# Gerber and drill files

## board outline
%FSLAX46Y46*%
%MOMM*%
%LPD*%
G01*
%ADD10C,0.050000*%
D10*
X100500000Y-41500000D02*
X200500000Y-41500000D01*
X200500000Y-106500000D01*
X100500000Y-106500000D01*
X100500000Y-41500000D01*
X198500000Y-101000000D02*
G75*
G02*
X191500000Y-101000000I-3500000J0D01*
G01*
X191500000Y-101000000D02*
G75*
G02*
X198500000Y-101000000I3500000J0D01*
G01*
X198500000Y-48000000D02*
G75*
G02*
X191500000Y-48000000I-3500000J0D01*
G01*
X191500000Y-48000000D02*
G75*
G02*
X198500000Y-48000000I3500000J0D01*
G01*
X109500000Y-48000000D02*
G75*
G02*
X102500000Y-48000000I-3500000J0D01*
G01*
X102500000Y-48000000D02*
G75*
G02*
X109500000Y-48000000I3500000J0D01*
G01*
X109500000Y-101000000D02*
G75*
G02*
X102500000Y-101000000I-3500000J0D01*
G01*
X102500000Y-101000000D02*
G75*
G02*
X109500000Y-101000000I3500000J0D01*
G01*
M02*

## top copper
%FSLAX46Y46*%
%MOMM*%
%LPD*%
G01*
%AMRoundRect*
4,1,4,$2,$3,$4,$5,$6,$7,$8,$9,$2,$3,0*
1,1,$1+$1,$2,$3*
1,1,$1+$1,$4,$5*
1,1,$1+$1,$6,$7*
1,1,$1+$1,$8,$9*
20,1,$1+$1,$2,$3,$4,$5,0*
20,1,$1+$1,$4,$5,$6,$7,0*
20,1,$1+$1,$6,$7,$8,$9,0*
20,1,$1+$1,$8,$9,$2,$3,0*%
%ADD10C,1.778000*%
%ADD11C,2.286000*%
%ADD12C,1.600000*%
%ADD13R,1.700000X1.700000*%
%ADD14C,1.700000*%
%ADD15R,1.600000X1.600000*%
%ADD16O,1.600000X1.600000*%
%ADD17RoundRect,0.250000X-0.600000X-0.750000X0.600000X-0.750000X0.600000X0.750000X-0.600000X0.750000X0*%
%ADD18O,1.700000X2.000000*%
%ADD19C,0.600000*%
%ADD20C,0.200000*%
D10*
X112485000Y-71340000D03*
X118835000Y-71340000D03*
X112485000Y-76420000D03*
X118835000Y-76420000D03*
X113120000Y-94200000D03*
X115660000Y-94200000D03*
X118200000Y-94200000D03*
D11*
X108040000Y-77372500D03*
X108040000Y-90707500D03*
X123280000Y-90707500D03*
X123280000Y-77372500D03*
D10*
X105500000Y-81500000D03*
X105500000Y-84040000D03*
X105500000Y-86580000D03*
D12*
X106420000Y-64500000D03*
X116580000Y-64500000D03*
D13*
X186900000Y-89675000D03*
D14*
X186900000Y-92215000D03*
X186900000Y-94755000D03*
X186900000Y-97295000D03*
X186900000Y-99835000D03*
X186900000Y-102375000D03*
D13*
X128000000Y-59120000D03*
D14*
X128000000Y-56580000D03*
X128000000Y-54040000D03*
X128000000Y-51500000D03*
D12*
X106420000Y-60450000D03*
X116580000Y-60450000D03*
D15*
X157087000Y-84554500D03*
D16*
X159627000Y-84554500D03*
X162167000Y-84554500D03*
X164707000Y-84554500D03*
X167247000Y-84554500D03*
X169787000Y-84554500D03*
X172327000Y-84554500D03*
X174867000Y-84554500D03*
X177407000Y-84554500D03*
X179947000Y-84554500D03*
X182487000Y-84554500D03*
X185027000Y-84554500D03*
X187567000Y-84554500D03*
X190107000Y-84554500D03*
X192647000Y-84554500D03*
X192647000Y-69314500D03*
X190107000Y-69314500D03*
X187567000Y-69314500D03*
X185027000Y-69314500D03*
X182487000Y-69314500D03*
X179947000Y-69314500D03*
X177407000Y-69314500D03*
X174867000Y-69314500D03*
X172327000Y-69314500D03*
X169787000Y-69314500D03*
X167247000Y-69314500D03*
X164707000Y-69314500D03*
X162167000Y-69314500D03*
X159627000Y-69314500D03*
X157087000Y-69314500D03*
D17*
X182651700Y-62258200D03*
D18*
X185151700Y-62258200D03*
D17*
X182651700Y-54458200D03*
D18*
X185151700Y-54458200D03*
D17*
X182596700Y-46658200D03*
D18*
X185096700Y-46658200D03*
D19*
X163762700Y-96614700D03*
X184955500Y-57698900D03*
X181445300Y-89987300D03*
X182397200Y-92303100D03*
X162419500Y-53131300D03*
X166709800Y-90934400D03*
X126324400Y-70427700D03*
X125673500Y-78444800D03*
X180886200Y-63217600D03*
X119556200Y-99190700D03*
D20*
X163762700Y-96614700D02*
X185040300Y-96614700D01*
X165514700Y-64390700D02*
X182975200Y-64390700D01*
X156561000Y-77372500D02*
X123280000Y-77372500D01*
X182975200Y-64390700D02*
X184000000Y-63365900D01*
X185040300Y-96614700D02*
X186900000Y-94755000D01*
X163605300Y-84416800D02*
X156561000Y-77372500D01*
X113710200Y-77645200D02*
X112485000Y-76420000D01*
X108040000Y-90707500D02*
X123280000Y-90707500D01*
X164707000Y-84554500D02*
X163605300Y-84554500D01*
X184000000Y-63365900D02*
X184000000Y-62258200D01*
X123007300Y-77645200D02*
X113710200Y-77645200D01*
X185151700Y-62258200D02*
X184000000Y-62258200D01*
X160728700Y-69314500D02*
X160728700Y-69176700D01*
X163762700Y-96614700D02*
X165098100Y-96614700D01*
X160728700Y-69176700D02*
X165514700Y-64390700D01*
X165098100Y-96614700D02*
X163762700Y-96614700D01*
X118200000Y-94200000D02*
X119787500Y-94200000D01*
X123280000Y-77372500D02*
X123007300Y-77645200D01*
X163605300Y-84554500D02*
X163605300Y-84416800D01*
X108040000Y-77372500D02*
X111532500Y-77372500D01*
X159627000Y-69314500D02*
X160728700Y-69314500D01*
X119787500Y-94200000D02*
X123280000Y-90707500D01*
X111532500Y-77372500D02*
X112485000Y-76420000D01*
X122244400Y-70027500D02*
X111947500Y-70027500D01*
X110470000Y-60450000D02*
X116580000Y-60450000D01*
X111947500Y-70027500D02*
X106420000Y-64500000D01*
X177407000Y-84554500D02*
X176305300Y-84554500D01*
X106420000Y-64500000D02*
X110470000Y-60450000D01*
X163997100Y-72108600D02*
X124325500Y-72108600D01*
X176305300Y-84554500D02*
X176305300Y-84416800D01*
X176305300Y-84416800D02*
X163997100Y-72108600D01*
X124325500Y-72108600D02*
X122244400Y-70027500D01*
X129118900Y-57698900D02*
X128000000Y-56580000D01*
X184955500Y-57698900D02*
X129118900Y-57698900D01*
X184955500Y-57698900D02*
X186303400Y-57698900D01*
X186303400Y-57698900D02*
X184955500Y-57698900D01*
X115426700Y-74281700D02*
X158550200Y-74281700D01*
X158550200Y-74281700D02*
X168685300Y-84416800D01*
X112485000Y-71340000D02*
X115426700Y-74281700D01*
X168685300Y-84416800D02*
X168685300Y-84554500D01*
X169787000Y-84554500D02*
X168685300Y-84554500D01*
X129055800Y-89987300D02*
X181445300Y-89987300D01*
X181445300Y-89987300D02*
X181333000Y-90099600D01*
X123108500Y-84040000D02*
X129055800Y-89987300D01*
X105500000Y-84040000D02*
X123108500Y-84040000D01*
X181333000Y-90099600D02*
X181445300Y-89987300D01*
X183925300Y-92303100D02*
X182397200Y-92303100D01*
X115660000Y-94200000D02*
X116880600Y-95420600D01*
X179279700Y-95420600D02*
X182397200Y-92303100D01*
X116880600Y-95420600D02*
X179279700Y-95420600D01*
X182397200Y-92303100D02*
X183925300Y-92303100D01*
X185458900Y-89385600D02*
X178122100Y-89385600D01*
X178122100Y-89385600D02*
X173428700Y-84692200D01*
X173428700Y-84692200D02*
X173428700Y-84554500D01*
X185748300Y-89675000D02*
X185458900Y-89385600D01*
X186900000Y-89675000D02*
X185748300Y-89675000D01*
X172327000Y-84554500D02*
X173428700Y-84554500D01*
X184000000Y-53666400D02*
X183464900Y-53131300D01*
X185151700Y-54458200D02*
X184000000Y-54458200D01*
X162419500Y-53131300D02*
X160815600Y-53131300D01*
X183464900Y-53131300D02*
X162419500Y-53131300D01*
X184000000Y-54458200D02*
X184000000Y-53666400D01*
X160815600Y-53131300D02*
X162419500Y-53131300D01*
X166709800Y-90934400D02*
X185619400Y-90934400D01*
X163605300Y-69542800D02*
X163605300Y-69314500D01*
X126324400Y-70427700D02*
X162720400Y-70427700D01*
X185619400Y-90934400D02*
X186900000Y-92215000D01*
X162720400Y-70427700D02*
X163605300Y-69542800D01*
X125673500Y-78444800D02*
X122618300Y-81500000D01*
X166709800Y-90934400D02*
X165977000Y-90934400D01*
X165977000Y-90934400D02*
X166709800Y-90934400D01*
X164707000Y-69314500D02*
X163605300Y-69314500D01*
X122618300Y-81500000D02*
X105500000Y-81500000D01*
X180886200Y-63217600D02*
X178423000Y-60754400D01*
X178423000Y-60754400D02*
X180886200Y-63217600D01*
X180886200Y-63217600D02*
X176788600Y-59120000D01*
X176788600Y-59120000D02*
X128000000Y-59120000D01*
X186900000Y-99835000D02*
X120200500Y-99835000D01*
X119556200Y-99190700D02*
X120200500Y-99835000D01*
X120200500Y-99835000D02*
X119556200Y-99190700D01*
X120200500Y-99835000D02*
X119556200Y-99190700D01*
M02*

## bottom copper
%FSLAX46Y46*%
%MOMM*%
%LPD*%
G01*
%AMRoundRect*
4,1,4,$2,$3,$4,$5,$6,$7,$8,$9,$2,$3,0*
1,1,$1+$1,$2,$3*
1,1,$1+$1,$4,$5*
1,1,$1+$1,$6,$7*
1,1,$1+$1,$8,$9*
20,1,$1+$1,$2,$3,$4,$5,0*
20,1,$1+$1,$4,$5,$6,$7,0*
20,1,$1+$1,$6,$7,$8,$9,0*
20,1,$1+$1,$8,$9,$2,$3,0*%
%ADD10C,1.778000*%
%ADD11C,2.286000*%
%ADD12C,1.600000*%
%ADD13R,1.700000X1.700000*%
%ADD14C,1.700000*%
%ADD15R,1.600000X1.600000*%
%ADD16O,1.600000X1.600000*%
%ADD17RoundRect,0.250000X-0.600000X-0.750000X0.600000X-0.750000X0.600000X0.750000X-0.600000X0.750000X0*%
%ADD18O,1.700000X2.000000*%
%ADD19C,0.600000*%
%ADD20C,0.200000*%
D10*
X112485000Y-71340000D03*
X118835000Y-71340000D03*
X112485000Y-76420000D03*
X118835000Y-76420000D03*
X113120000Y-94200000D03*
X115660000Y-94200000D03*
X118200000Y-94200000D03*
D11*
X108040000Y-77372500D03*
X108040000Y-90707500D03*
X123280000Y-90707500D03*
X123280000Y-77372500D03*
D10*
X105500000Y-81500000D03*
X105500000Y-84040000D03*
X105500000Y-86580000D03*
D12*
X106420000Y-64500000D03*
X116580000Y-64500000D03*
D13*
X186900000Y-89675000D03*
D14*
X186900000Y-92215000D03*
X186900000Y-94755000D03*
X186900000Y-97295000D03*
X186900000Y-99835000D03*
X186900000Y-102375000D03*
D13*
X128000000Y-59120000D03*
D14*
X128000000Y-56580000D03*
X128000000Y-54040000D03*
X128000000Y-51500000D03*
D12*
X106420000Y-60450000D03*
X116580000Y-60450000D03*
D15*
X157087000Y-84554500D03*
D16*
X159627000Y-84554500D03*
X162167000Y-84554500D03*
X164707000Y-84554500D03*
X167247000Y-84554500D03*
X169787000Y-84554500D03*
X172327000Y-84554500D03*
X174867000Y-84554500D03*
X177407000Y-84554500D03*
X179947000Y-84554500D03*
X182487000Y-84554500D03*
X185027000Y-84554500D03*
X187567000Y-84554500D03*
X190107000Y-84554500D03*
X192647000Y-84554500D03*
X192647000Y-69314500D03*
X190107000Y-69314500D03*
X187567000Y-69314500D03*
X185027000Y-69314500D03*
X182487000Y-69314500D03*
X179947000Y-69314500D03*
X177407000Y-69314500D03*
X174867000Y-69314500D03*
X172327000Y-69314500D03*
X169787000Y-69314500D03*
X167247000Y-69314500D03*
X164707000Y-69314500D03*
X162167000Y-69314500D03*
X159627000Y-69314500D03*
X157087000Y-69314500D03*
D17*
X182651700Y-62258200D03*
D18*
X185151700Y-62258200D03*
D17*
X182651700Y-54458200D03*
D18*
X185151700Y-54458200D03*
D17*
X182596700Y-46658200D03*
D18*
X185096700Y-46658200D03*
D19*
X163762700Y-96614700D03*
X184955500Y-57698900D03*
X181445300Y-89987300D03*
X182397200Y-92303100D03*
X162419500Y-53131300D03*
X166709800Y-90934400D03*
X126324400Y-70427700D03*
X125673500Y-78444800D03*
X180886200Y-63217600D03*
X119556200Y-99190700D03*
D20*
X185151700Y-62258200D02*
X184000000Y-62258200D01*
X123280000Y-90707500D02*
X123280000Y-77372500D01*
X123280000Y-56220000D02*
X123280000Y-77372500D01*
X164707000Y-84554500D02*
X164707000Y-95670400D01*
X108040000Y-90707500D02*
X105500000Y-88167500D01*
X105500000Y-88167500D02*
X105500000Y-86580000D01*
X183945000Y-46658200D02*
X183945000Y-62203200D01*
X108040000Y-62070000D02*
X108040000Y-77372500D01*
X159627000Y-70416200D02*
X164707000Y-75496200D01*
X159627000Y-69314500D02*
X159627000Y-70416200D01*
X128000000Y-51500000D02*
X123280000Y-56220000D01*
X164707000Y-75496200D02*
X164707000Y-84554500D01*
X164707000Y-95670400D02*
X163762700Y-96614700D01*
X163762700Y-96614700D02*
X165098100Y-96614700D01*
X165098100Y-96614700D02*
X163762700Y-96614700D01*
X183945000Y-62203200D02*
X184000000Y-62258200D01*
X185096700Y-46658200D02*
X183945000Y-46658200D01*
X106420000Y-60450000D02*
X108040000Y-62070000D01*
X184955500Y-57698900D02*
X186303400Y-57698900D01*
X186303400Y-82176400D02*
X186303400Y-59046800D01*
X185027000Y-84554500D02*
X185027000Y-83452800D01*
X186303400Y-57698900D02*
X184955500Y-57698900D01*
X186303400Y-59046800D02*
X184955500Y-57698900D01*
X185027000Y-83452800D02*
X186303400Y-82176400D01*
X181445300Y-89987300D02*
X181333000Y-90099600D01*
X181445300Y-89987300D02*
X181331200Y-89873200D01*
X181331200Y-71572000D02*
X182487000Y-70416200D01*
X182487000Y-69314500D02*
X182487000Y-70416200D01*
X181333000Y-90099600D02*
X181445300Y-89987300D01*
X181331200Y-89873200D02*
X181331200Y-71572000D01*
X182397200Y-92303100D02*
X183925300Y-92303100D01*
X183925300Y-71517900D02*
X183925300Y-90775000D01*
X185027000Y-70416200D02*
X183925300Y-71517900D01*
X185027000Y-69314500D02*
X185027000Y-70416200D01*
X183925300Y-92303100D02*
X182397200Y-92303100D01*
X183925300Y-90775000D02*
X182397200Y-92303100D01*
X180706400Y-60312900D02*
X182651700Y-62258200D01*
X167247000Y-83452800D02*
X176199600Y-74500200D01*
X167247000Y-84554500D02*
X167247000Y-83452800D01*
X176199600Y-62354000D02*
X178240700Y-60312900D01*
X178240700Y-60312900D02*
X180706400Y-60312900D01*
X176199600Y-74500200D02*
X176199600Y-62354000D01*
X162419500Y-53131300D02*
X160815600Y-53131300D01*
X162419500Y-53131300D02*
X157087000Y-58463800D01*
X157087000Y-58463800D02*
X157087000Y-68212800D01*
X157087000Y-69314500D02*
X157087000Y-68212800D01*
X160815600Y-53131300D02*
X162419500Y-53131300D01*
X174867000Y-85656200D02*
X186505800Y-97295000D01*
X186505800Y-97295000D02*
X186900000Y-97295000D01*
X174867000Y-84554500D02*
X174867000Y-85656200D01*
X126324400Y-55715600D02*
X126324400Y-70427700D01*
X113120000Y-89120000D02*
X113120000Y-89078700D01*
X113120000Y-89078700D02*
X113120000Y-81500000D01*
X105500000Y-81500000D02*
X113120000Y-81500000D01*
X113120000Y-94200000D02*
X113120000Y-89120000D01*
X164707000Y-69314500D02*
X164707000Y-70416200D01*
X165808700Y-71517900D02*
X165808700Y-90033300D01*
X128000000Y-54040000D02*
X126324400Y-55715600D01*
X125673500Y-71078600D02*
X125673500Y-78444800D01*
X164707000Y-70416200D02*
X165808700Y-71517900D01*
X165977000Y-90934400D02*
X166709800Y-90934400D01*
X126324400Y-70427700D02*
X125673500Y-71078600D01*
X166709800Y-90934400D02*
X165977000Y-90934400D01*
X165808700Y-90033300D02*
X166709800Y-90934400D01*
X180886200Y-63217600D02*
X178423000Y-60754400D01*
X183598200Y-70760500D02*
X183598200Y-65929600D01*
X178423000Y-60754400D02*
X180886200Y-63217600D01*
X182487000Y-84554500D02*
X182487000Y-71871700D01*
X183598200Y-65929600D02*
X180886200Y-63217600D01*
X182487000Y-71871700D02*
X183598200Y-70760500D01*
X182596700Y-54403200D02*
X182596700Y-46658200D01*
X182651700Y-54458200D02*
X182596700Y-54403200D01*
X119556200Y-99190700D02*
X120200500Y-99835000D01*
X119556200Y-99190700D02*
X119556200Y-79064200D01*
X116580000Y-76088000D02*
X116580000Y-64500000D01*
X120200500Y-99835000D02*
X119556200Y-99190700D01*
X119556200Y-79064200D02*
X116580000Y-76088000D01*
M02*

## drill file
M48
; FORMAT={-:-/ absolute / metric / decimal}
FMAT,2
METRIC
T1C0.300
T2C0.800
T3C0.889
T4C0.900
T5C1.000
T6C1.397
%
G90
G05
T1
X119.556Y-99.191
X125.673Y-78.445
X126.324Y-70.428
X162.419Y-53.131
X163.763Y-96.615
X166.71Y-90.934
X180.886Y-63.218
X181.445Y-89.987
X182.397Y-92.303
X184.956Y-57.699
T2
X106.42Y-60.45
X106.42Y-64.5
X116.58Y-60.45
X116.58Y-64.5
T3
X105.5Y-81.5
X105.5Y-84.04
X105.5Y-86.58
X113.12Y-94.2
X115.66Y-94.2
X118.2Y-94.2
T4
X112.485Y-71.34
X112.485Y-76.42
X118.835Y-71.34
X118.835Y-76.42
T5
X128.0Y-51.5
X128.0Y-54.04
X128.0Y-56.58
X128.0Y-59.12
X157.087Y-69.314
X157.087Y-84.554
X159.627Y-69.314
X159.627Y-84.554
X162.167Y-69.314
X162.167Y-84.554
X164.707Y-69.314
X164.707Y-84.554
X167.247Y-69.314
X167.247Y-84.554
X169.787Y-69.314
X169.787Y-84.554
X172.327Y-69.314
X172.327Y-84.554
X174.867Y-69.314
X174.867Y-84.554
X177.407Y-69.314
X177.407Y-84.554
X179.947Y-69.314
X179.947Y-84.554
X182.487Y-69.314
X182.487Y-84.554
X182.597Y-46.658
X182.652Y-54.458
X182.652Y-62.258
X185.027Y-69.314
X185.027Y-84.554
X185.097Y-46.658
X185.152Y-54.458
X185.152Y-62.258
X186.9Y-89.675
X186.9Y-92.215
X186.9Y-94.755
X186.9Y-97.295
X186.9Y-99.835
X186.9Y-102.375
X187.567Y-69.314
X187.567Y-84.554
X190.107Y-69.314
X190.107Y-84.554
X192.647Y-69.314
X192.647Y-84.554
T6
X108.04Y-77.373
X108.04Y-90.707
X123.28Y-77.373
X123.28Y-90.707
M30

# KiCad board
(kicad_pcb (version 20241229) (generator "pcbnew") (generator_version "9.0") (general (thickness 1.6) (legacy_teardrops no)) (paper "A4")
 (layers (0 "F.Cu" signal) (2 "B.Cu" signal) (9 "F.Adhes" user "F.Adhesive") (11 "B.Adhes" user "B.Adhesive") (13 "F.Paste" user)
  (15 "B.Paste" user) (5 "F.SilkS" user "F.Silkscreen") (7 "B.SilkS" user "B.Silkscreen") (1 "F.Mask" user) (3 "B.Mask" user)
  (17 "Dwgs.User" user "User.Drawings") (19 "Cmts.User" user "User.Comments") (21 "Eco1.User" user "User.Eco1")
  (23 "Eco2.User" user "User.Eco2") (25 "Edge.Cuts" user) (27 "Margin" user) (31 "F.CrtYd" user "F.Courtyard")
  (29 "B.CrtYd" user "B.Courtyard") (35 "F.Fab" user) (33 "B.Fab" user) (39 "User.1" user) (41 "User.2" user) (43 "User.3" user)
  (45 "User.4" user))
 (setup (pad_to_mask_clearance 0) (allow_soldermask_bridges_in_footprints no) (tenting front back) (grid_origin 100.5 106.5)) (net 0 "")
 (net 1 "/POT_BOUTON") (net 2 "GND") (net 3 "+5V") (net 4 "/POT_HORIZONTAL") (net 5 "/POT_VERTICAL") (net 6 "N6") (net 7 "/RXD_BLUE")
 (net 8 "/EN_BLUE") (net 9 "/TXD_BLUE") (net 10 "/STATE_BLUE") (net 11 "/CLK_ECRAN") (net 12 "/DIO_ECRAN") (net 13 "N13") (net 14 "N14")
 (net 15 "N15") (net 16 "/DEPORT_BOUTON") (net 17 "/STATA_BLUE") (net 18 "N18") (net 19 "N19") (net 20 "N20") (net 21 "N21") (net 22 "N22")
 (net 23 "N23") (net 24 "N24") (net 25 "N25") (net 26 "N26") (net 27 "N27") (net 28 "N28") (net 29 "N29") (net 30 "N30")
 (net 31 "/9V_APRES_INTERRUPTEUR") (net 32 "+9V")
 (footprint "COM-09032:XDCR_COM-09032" (layer "F.Cu") (at 115.66 84.04)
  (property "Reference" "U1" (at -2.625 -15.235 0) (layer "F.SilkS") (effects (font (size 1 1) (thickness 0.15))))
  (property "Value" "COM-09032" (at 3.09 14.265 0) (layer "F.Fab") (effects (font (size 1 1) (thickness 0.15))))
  (pad "B1A" thru_hole circle (at -3.175 -12.7) (size 1.778 1.778) (drill 0.9) (layers "*.Cu" "*.Mask") (remove_unused_layers no)
   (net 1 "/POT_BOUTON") (solder_mask_margin 0.102))
  (pad "B1B" thru_hole circle (at 3.175 -12.7) (size 1.778 1.778) (drill 0.9) (layers "*.Cu" "*.Mask") (remove_unused_layers no)
   (solder_mask_margin 0.102))
  (pad "B2A" thru_hole circle (at -3.175 -7.62) (size 1.778 1.778) (drill 0.9) (layers "*.Cu" "*.Mask") (remove_unused_layers no)
   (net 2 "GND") (solder_mask_margin 0.102))
  (pad "B2B" thru_hole circle (at 3.175 -7.62) (size 1.778 1.778) (drill 0.9) (layers "*.Cu" "*.Mask") (remove_unused_layers no)
   (solder_mask_margin 0.102))
  (pad "H1" thru_hole circle (at -2.54 10.16) (size 1.778 1.778) (drill 0.889) (layers "*.Cu" "*.Mask") (remove_unused_layers no)
   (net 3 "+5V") (solder_mask_margin 0.102))
  (pad "H2" thru_hole circle (at 0 10.16) (size 1.778 1.778) (drill 0.889) (layers "*.Cu" "*.Mask") (remove_unused_layers no)
   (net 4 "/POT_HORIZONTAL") (solder_mask_margin 0.102))
  (pad "H3" thru_hole circle (at 2.54 10.16) (size 1.778 1.778) (drill 0.889) (layers "*.Cu" "*.Mask") (remove_unused_layers no)
   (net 2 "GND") (solder_mask_margin 0.102))
  (pad "S1" thru_hole circle (at -7.62 -6.6675) (size 2.286 2.286) (drill 1.397) (layers "*.Cu" "*.Mask") (remove_unused_layers no)
   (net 2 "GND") (solder_mask_margin 0.102))
  (pad "S2" thru_hole circle (at -7.62 6.6675) (size 2.286 2.286) (drill 1.397) (layers "*.Cu" "*.Mask") (remove_unused_layers no)
   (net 2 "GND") (solder_mask_margin 0.102))
  (pad "S3" thru_hole circle (at 7.62 6.6675) (size 2.286 2.286) (drill 1.397) (layers "*.Cu" "*.Mask") (remove_unused_layers no)
   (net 2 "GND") (solder_mask_margin 0.102))
  (pad "S4" thru_hole circle (at 7.62 -6.6675) (size 2.286 2.286) (drill 1.397) (layers "*.Cu" "*.Mask") (remove_unused_layers no)
   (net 2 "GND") (solder_mask_margin 0.102))
  (pad "V1" thru_hole circle (at -10.16 -2.54) (size 1.778 1.778) (drill 0.889) (layers "*.Cu" "*.Mask") (remove_unused_layers no)
   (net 3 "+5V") (solder_mask_margin 0.102))
  (pad "V2" thru_hole circle (at -10.16 0) (size 1.778 1.778) (drill 0.889) (layers "*.Cu" "*.Mask") (remove_unused_layers no)
   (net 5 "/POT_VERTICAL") (solder_mask_margin 0.102))
  (pad "V3" thru_hole circle (at -10.16 2.54) (size 1.778 1.778) (drill 0.889) (layers "*.Cu" "*.Mask") (remove_unused_layers no)
   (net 2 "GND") (solder_mask_margin 0.102)))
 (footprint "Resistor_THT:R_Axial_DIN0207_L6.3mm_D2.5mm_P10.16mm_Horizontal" (layer "F.Cu") (at 106.42 64.5)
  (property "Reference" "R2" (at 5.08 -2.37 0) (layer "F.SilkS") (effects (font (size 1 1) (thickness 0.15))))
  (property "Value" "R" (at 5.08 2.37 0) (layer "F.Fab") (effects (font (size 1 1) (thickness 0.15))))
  (pad "1" thru_hole circle (at 0 0) (size 1.6 1.6) (drill 0.8) (layers "*.Cu" "*.Mask") (remove_unused_layers no) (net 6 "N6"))
  (pad "2" thru_hole circle (at 10.16 0) (size 1.6 1.6) (drill 0.8) (layers "*.Cu" "*.Mask") (remove_unused_layers no) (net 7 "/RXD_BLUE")))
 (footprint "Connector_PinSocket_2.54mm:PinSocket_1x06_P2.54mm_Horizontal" (layer "F.Cu") (at 186.9 89.675)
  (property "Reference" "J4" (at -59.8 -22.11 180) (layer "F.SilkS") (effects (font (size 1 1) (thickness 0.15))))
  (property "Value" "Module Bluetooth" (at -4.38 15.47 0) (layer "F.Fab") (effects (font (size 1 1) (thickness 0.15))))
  (pad "1" thru_hole rect (at 0 0) (size 1.7 1.7) (drill 1) (layers "*.Cu" "*.Mask") (remove_unused_layers no) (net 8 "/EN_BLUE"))
  (pad "2" thru_hole circle (at 0 2.54) (size 1.7 1.7) (drill 1) (layers "*.Cu" "*.Mask") (remove_unused_layers no) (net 3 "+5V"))
  (pad "3" thru_hole circle (at 0 5.08) (size 1.7 1.7) (drill 1) (layers "*.Cu" "*.Mask") (remove_unused_layers no) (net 2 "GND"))
  (pad "4" thru_hole circle (at 0 7.62) (size 1.7 1.7) (drill 1) (layers "*.Cu" "*.Mask") (remove_unused_layers no) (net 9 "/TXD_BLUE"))
  (pad "5" thru_hole circle (at 0 10.16) (size 1.7 1.7) (drill 1) (layers "*.Cu" "*.Mask") (remove_unused_layers no) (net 7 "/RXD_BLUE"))
  (pad "6" thru_hole circle (at 0 12.7) (size 1.7 1.7) (drill 1) (layers "*.Cu" "*.Mask") (remove_unused_layers no) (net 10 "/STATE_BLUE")))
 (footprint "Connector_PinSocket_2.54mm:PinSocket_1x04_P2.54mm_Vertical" (layer "F.Cu") (at 128 59.12 180)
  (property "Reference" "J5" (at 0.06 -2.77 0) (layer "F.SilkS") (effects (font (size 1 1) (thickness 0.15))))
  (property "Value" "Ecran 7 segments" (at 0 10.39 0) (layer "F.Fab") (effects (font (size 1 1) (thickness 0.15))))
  (pad "1" thru_hole rect (at 0 0 180) (size 1.7 1.7) (drill 1) (layers "*.Cu" "*.Mask") (remove_unused_layers no) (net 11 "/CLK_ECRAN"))
  (pad "2" thru_hole circle (at 0 2.54 180) (size 1.7 1.7) (drill 1) (layers "*.Cu" "*.Mask") (remove_unused_layers no)
   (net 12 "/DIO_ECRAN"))
  (pad "3" thru_hole circle (at 0 5.08 180) (size 1.7 1.7) (drill 1) (layers "*.Cu" "*.Mask") (remove_unused_layers no) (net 3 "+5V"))
  (pad "4" thru_hole circle (at 0 7.62 180) (size 1.7 1.7) (drill 1) (layers "*.Cu" "*.Mask") (remove_unused_layers no) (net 2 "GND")))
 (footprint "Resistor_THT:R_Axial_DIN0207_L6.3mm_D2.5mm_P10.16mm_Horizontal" (layer "F.Cu") (at 106.42 60.45)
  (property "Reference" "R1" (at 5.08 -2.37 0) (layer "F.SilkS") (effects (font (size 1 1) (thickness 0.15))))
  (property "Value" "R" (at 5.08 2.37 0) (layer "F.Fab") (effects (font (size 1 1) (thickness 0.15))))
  (pad "1" thru_hole circle (at 0 0) (size 1.6 1.6) (drill 0.8) (layers "*.Cu" "*.Mask") (remove_unused_layers no) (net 2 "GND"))
  (pad "2" thru_hole circle (at 10.16 0) (size 1.6 1.6) (drill 0.8) (layers "*.Cu" "*.Mask") (remove_unused_layers no) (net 6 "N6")))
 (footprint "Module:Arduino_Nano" (layer "F.Cu") (at 157.087 84.5545 90)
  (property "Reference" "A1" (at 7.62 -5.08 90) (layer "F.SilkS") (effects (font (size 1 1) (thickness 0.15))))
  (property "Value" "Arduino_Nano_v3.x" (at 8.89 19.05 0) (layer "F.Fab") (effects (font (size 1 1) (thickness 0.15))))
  (pad "1" thru_hole rect (at 0 0 90) (size 1.6 1.6) (drill 1) (layers "*.Cu" "*.Mask") (remove_unused_layers no) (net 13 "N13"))
  (pad "2" thru_hole oval (at 0 2.54 90) (size 1.6 1.6) (drill 1) (layers "*.Cu" "*.Mask") (remove_unused_layers no) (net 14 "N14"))
  (pad "3" thru_hole oval (at 0 5.08 90) (size 1.6 1.6) (drill 1) (layers "*.Cu" "*.Mask") (remove_unused_layers no) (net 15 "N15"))
  (pad "4" thru_hole oval (at 0 7.62 90) (size 1.6 1.6) (drill 1) (layers "*.Cu" "*.Mask") (remove_unused_layers no) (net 2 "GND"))
  (pad "5" thru_hole oval (at 0 10.16 90) (size 1.6 1.6) (drill 1) (layers "*.Cu" "*.Mask") (remove_unused_layers no)
   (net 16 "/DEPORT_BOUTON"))
  (pad "6" thru_hole oval (at 0 12.7 90) (size 1.6 1.6) (drill 1) (layers "*.Cu" "*.Mask") (remove_unused_layers no) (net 1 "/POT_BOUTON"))
  (pad "7" thru_hole oval (at 0 15.24 90) (size 1.6 1.6) (drill 1) (layers "*.Cu" "*.Mask") (remove_unused_layers no) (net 8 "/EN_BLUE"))
  (pad "8" thru_hole oval (at 0 17.78 90) (size 1.6 1.6) (drill 1) (layers "*.Cu" "*.Mask") (remove_unused_layers no) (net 9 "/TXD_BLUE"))
  (pad "9" thru_hole oval (at 0 20.32 90) (size 1.6 1.6) (drill 1) (layers "*.Cu" "*.Mask") (remove_unused_layers no) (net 6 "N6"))
  (pad "10" thru_hole oval (at 0 22.86 90) (size 1.6 1.6) (drill 1) (layers "*.Cu" "*.Mask") (remove_unused_layers no)
   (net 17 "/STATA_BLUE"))
  (pad "11" thru_hole oval (at 0 25.4 90) (size 1.6 1.6) (drill 1) (layers "*.Cu" "*.Mask") (remove_unused_layers no) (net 11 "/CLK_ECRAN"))
  (pad "12" thru_hole oval (at 0 27.94 90) (size 1.6 1.6) (drill 1) (layers "*.Cu" "*.Mask") (remove_unused_layers no) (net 12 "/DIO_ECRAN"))
  (pad "13" thru_hole oval (at 0 30.48 90) (size 1.6 1.6) (drill 1) (layers "*.Cu" "*.Mask") (remove_unused_layers no) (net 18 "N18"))
  (pad "14" thru_hole oval (at 0 33.02 90) (size 1.6 1.6) (drill 1) (layers "*.Cu" "*.Mask") (remove_unused_layers no) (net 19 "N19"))
  (pad "15" thru_hole oval (at 0 35.56 90) (size 1.6 1.6) (drill 1) (layers "*.Cu" "*.Mask") (remove_unused_layers no) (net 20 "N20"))
  (pad "16" thru_hole oval (at 15.24 35.56 90) (size 1.6 1.6) (drill 1) (layers "*.Cu" "*.Mask") (remove_unused_layers no) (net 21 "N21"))
  (pad "17" thru_hole oval (at 15.24 33.02 90) (size 1.6 1.6) (drill 1) (layers "*.Cu" "*.Mask") (remove_unused_layers no) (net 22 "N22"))
  (pad "18" thru_hole oval (at 15.24 30.48 90) (size 1.6 1.6) (drill 1) (layers "*.Cu" "*.Mask") (remove_unused_layers no) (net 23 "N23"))
  (pad "19" thru_hole oval (at 15.24 27.94 90) (size 1.6 1.6) (drill 1) (layers "*.Cu" "*.Mask") (remove_unused_layers no)
   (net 4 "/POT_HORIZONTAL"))
  (pad "20" thru_hole oval (at 15.24 25.4 90) (size 1.6 1.6) (drill 1) (layers "*.Cu" "*.Mask") (remove_unused_layers no)
   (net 5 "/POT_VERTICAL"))
  (pad "21" thru_hole oval (at 15.24 22.86 90) (size 1.6 1.6) (drill 1) (layers "*.Cu" "*.Mask") (remove_unused_layers no) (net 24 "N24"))
  (pad "22" thru_hole oval (at 15.24 20.32 90) (size 1.6 1.6) (drill 1) (layers "*.Cu" "*.Mask") (remove_unused_layers no) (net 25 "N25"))
  (pad "23" thru_hole oval (at 15.24 17.78 90) (size 1.6 1.6) (drill 1) (layers "*.Cu" "*.Mask") (remove_unused_layers no) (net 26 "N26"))
  (pad "24" thru_hole oval (at 15.24 15.24 90) (size 1.6 1.6) (drill 1) (layers "*.Cu" "*.Mask") (remove_unused_layers no) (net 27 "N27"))
  (pad "25" thru_hole oval (at 15.24 12.7 90) (size 1.6 1.6) (drill 1) (layers "*.Cu" "*.Mask") (remove_unused_layers no) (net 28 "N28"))
  (pad "26" thru_hole oval (at 15.24 10.16 90) (size 1.6 1.6) (drill 1) (layers "*.Cu" "*.Mask") (remove_unused_layers no) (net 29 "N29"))
  (pad "27" thru_hole oval (at 15.24 7.62 90) (size 1.6 1.6) (drill 1) (layers "*.Cu" "*.Mask") (remove_unused_layers no) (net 3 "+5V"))
  (pad "28" thru_hole oval (at 15.24 5.08 90) (size 1.6 1.6) (drill 1) (layers "*.Cu" "*.Mask") (remove_unused_layers no) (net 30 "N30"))
  (pad "29" thru_hole oval (at 15.24 2.54 90) (size 1.6 1.6) (drill 1) (layers "*.Cu" "*.Mask") (remove_unused_layers no) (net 2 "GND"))
  (pad "30" thru_hole oval (at 15.24 0 90) (size 1.6 1.6) (drill 1) (layers "*.Cu" "*.Mask") (remove_unused_layers no)
   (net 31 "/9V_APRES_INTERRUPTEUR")))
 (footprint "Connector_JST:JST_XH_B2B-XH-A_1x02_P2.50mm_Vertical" (layer "F.Cu") (at 182.6517 62.2582)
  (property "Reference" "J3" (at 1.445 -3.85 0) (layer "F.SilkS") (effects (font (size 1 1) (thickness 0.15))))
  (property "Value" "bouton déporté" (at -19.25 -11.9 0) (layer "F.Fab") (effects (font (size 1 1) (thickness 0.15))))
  (pad "1" thru_hole roundrect (at 0 0) (size 1.7 2) (drill 1) (layers "*.Cu" "*.Mask") (remove_unused_layers no)
   (roundrect_rratio 0.147059) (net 16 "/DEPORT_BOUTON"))
  (pad "2" thru_hole oval (at 2.5 0) (size 1.7 2) (drill 1) (layers "*.Cu" "*.Mask") (remove_unused_layers no) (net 2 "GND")))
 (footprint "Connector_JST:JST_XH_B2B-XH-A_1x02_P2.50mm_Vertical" (layer "F.Cu") (at 182.6517 54.4582)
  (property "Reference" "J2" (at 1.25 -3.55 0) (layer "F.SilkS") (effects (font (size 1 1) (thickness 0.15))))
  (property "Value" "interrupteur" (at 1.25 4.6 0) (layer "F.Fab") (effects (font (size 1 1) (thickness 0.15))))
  (pad "1" thru_hole roundrect (at 0 0) (size 1.7 2) (drill 1) (layers "*.Cu" "*.Mask") (remove_unused_layers no)
   (roundrect_rratio 0.147059) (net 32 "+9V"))
  (pad "2" thru_hole oval (at 2.5 0) (size 1.7 2) (drill 1) (layers "*.Cu" "*.Mask") (remove_unused_layers no)
   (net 31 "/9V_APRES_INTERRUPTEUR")))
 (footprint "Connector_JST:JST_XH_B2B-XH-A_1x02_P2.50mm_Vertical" (layer "F.Cu") (at 182.5967 46.6582)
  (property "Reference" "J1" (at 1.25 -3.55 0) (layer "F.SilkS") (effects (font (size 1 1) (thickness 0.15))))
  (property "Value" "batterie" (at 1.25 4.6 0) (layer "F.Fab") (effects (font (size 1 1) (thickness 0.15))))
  (pad "1" thru_hole roundrect (at 0 0) (size 1.7 2) (drill 1) (layers "*.Cu" "*.Mask") (remove_unused_layers no)
   (roundrect_rratio 0.147059) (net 32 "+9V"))
  (pad "2" thru_hole oval (at 2.5 0) (size 1.7 2) (drill 1) (layers "*.Cu" "*.Mask") (remove_unused_layers no) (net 2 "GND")))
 (gr_rect (start 100.5 41.5) (end 200.5 106.5) (stroke (width 0.05) (type solid)) (fill no) (layer "Edge.Cuts"))
 (gr_circle (center 195 101) (end 198.5 101) (stroke (width 0.05) (type solid)) (fill no) (layer "Edge.Cuts"))
 (gr_circle (center 195 48) (end 198.5 48) (stroke (width 0.05) (type solid)) (fill no) (layer "Edge.Cuts"))
 (gr_circle (center 106 48) (end 109.5 48) (stroke (width 0.05) (type solid)) (fill no) (layer "Edge.Cuts"))
 (gr_circle (center 106 101) (end 109.5 101) (stroke (width 0.05) (type solid)) (fill no) (layer "Edge.Cuts"))
 (segment (start 163.7627 96.6147) (end 185.0403 96.6147) (width 0.2) (layer "F.Cu") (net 2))
 (segment (start 165.5147 64.3907) (end 182.9752 64.3907) (width 0.2) (layer "F.Cu") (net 2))
 (segment (start 156.561 77.3725) (end 123.28 77.3725) (width 0.2) (layer "F.Cu") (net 2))
 (segment (start 182.9752 64.3907) (end 184 63.3659) (width 0.2) (layer "F.Cu") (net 2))
 (segment (start 185.0403 96.6147) (end 186.9 94.755) (width 0.2) (layer "F.Cu") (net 2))
 (segment (start 163.6053 84.4168) (end 156.561 77.3725) (width 0.2) (layer "F.Cu") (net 2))
 (segment (start 113.7102 77.6452) (end 112.485 76.42) (width 0.2) (layer "F.Cu") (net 2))
 (segment (start 108.04 90.7075) (end 123.28 90.7075) (width 0.2) (layer "F.Cu") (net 2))
 (segment (start 164.707 84.5545) (end 163.6053 84.5545) (width 0.2) (layer "F.Cu") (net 2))
 (segment (start 184 63.3659) (end 184 62.2582) (width 0.2) (layer "F.Cu") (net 2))
 (segment (start 123.0073 77.6452) (end 113.7102 77.6452) (width 0.2) (layer "F.Cu") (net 2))
 (segment (start 185.1517 62.2582) (end 184 62.2582) (width 0.2) (layer "F.Cu") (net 2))
 (segment (start 160.7287 69.3145) (end 160.7287 69.1767) (width 0.2) (layer "F.Cu") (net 2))
 (segment (start 163.7627 96.6147) (end 165.0981 96.6147) (width 0.2) (layer "F.Cu") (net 2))
 (segment (start 160.7287 69.1767) (end 165.5147 64.3907) (width 0.2) (layer "F.Cu") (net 2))
 (segment (start 165.0981 96.6147) (end 163.7627 96.6147) (width 0.2) (layer "F.Cu") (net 2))
 (segment (start 118.2 94.2) (end 119.7875 94.2) (width 0.2) (layer "F.Cu") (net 2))
 (segment (start 123.28 77.3725) (end 123.0073 77.6452) (width 0.2) (layer "F.Cu") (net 2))
 (segment (start 163.6053 84.5545) (end 163.6053 84.4168) (width 0.2) (layer "F.Cu") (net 2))
 (segment (start 108.04 77.3725) (end 111.5325 77.3725) (width 0.2) (layer "F.Cu") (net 2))
 (segment (start 159.627 69.3145) (end 160.7287 69.3145) (width 0.2) (layer "F.Cu") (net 2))
 (segment (start 119.7875 94.2) (end 123.28 90.7075) (width 0.2) (layer "F.Cu") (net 2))
 (segment (start 111.5325 77.3725) (end 112.485 76.42) (width 0.2) (layer "F.Cu") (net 2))
 (via (at 163.7627 96.6147) (size 0.6) (drill 0.3) (layers "F.Cu" "B.Cu") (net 2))
 (segment (start 185.1517 62.2582) (end 184 62.2582) (width 0.2) (layer "B.Cu") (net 2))
 (segment (start 123.28 90.7075) (end 123.28 77.3725) (width 0.2) (layer "B.Cu") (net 2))
 (segment (start 123.28 56.22) (end 123.28 77.3725) (width 0.2) (layer "B.Cu") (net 2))
 (segment (start 164.707 84.5545) (end 164.707 95.6704) (width 0.2) (layer "B.Cu") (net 2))
 (segment (start 108.04 90.7075) (end 105.5 88.1675) (width 0.2) (layer "B.Cu") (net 2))
 (segment (start 105.5 88.1675) (end 105.5 86.58) (width 0.2) (layer "B.Cu") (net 2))
 (segment (start 183.945 46.6582) (end 183.945 62.2032) (width 0.2) (layer "B.Cu") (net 2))
 (segment (start 108.04 62.07) (end 108.04 77.3725) (width 0.2) (layer "B.Cu") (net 2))
 (segment (start 159.627 70.4162) (end 164.707 75.4962) (width 0.2) (layer "B.Cu") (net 2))
 (segment (start 159.627 69.3145) (end 159.627 70.4162) (width 0.2) (layer "B.Cu") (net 2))
 (segment (start 128 51.5) (end 123.28 56.22) (width 0.2) (layer "B.Cu") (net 2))
 (segment (start 164.707 75.4962) (end 164.707 84.5545) (width 0.2) (layer "B.Cu") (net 2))
 (segment (start 164.707 95.6704) (end 163.7627 96.6147) (width 0.2) (layer "B.Cu") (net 2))
 (segment (start 163.7627 96.6147) (end 165.0981 96.6147) (width 0.2) (layer "B.Cu") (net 2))
 (segment (start 165.0981 96.6147) (end 163.7627 96.6147) (width 0.2) (layer "B.Cu") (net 2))
 (segment (start 183.945 62.2032) (end 184 62.2582) (width 0.2) (layer "B.Cu") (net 2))
 (segment (start 185.0967 46.6582) (end 183.945 46.6582) (width 0.2) (layer "B.Cu") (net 2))
 (segment (start 106.42 60.45) (end 108.04 62.07) (width 0.2) (layer "B.Cu") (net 2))
 (segment (start 122.2444 70.0275) (end 111.9475 70.0275) (width 0.2) (layer "F.Cu") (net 6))
 (segment (start 110.47 60.45) (end 116.58 60.45) (width 0.2) (layer "F.Cu") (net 6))
 (segment (start 111.9475 70.0275) (end 106.42 64.5) (width 0.2) (layer "F.Cu") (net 6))
 (segment (start 177.407 84.5545) (end 176.3053 84.5545) (width 0.2) (layer "F.Cu") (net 6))
 (segment (start 106.42 64.5) (end 110.47 60.45) (width 0.2) (layer "F.Cu") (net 6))
 (segment (start 163.9971 72.1086) (end 124.3255 72.1086) (width 0.2) (layer "F.Cu") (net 6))
 (segment (start 176.3053 84.5545) (end 176.3053 84.4168) (width 0.2) (layer "F.Cu") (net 6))
 (segment (start 176.3053 84.4168) (end 163.9971 72.1086) (width 0.2) (layer "F.Cu") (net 6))
 (segment (start 124.3255 72.1086) (end 122.2444 70.0275) (width 0.2) (layer "F.Cu") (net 6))
 (segment (start 129.1189 57.6989) (end 128 56.58) (width 0.2) (layer "F.Cu") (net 12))
 (segment (start 184.9555 57.6989) (end 129.1189 57.6989) (width 0.2) (layer "F.Cu") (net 12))
 (segment (start 184.9555 57.6989) (end 186.3034 57.6989) (width 0.2) (layer "F.Cu") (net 12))
 (segment (start 186.3034 57.6989) (end 184.9555 57.6989) (width 0.2) (layer "F.Cu") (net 12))
 (via (at 184.9555 57.6989) (size 0.6) (drill 0.3) (layers "F.Cu" "B.Cu") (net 12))
 (segment (start 184.9555 57.6989) (end 186.3034 57.6989) (width 0.2) (layer "B.Cu") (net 12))
 (segment (start 186.3034 82.1764) (end 186.3034 59.0468) (width 0.2) (layer "B.Cu") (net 12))
 (segment (start 185.027 84.5545) (end 185.027 83.4528) (width 0.2) (layer "B.Cu") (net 12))
 (segment (start 186.3034 57.6989) (end 184.9555 57.6989) (width 0.2) (layer "B.Cu") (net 12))
 (segment (start 186.3034 59.0468) (end 184.9555 57.6989) (width 0.2) (layer "B.Cu") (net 12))
 (segment (start 185.027 83.4528) (end 186.3034 82.1764) (width 0.2) (layer "B.Cu") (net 12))
 (segment (start 115.4267 74.2817) (end 158.5502 74.2817) (width 0.2) (layer "F.Cu") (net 1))
 (segment (start 158.5502 74.2817) (end 168.6853 84.4168) (width 0.2) (layer "F.Cu") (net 1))
 (segment (start 112.485 71.34) (end 115.4267 74.2817) (width 0.2) (layer "F.Cu") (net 1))
 (segment (start 168.6853 84.4168) (end 168.6853 84.5545) (width 0.2) (layer "F.Cu") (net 1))
 (segment (start 169.787 84.5545) (end 168.6853 84.5545) (width 0.2) (layer "F.Cu") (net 1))
 (segment (start 129.0558 89.9873) (end 181.4453 89.9873) (width 0.2) (layer "F.Cu") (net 5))
 (segment (start 181.4453 89.9873) (end 181.333 90.0996) (width 0.2) (layer "F.Cu") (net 5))
 (segment (start 123.1085 84.04) (end 129.0558 89.9873) (width 0.2) (layer "F.Cu") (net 5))
 (segment (start 105.5 84.04) (end 123.1085 84.04) (width 0.2) (layer "F.Cu") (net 5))
 (segment (start 181.333 90.0996) (end 181.4453 89.9873) (width 0.2) (layer "F.Cu") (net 5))
 (via (at 181.4453 89.9873) (size 0.6) (drill 0.3) (layers "F.Cu" "B.Cu") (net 5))
 (segment (start 181.4453 89.9873) (end 181.333 90.0996) (width 0.2) (layer "B.Cu") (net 5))
 (segment (start 181.4453 89.9873) (end 181.3312 89.8732) (width 0.2) (layer "B.Cu") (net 5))
 (segment (start 181.3312 71.572) (end 182.487 70.4162) (width 0.2) (layer "B.Cu") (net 5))
 (segment (start 182.487 69.3145) (end 182.487 70.4162) (width 0.2) (layer "B.Cu") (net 5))
 (segment (start 181.333 90.0996) (end 181.4453 89.9873) (width 0.2) (layer "B.Cu") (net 5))
 (segment (start 181.3312 89.8732) (end 181.3312 71.572) (width 0.2) (layer "B.Cu") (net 5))
 (segment (start 183.9253 92.3031) (end 182.3972 92.3031) (width 0.2) (layer "F.Cu") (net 4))
 (segment (start 115.66 94.2) (end 116.8806 95.4206) (width 0.2) (layer "F.Cu") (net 4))
 (segment (start 179.2797 95.4206) (end 182.3972 92.3031) (width 0.2) (layer "F.Cu") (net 4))
 (segment (start 116.8806 95.4206) (end 179.2797 95.4206) (width 0.2) (layer "F.Cu") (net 4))
 (segment (start 182.3972 92.3031) (end 183.9253 92.3031) (width 0.2) (layer "F.Cu") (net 4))
 (via (at 182.3972 92.3031) (size 0.6) (drill 0.3) (layers "F.Cu" "B.Cu") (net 4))
 (segment (start 182.3972 92.3031) (end 183.9253 92.3031) (width 0.2) (layer "B.Cu") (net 4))
 (segment (start 183.9253 71.5179) (end 183.9253 90.775) (width 0.2) (layer "B.Cu") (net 4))
 (segment (start 185.027 70.4162) (end 183.9253 71.5179) (width 0.2) (layer "B.Cu") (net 4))
 (segment (start 185.027 69.3145) (end 185.027 70.4162) (width 0.2) (layer "B.Cu") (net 4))
 (segment (start 183.9253 92.3031) (end 182.3972 92.3031) (width 0.2) (layer "B.Cu") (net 4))
 (segment (start 183.9253 90.775) (end 182.3972 92.3031) (width 0.2) (layer "B.Cu") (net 4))
 (segment (start 185.4589 89.3856) (end 178.1221 89.3856) (width 0.2) (layer "F.Cu") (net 8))
 (segment (start 178.1221 89.3856) (end 173.4287 84.6922) (width 0.2) (layer "F.Cu") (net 8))
 (segment (start 173.4287 84.6922) (end 173.4287 84.5545) (width 0.2) (layer "F.Cu") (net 8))
 (segment (start 185.7483 89.675) (end 185.4589 89.3856) (width 0.2) (layer "F.Cu") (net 8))
 (segment (start 186.9 89.675) (end 185.7483 89.675) (width 0.2) (layer "F.Cu") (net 8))
 (segment (start 172.327 84.5545) (end 173.4287 84.5545) (width 0.2) (layer "F.Cu") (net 8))
 (segment (start 180.7064 60.3129) (end 182.6517 62.2582) (width 0.2) (layer "B.Cu") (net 16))
 (segment (start 167.247 83.4528) (end 176.1996 74.5002) (width 0.2) (layer "B.Cu") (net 16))
 (segment (start 167.247 84.5545) (end 167.247 83.4528) (width 0.2) (layer "B.Cu") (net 16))
 (segment (start 176.1996 62.354) (end 178.2407 60.3129) (width 0.2) (layer "B.Cu") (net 16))
 (segment (start 178.2407 60.3129) (end 180.7064 60.3129) (width 0.2) (layer "B.Cu") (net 16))
 (segment (start 176.1996 74.5002) (end 176.1996 62.354) (width 0.2) (layer "B.Cu") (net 16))
 (segment (start 184 53.6664) (end 183.4649 53.1313) (width 0.2) (layer "F.Cu") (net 31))
 (segment (start 185.1517 54.4582) (end 184 54.4582) (width 0.2) (layer "F.Cu") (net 31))
 (segment (start 162.4195 53.1313) (end 160.8156 53.1313) (width 0.2) (layer "F.Cu") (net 31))
 (segment (start 183.4649 53.1313) (end 162.4195 53.1313) (width 0.2) (layer "F.Cu") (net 31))
 (segment (start 184 54.4582) (end 184 53.6664) (width 0.2) (layer "F.Cu") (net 31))
 (segment (start 160.8156 53.1313) (end 162.4195 53.1313) (width 0.2) (layer "F.Cu") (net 31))
 (via (at 162.4195 53.1313) (size 0.6) (drill 0.3) (layers "F.Cu" "B.Cu") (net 31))
 (segment (start 162.4195 53.1313) (end 160.8156 53.1313) (width 0.2) (layer "B.Cu") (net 31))
 (segment (start 162.4195 53.1313) (end 157.087 58.4638) (width 0.2) (layer "B.Cu") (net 31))
 (segment (start 157.087 58.4638) (end 157.087 68.2128) (width 0.2) (layer "B.Cu") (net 31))
 (segment (start 157.087 69.3145) (end 157.087 68.2128) (width 0.2) (layer "B.Cu") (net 31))
 (segment (start 160.8156 53.1313) (end 162.4195 53.1313) (width 0.2) (layer "B.Cu") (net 31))
 (segment (start 174.867 85.6562) (end 186.5058 97.295) (width 0.2) (layer "B.Cu") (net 9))
 (segment (start 186.5058 97.295) (end 186.9 97.295) (width 0.2) (layer "B.Cu") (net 9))
 (segment (start 174.867 84.5545) (end 174.867 85.6562) (width 0.2) (layer "B.Cu") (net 9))
 (segment (start 166.7098 90.9344) (end 185.6194 90.9344) (width 0.2) (layer "F.Cu") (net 3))
 (segment (start 163.6053 69.5428) (end 163.6053 69.3145) (width 0.2) (layer "F.Cu") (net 3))
 (segment (start 126.3244 70.4277) (end 162.7204 70.4277) (width 0.2) (layer "F.Cu") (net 3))
 (segment (start 185.6194 90.9344) (end 186.9 92.215) (width 0.2) (layer "F.Cu") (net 3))
 (segment (start 162.7204 70.4277) (end 163.6053 69.5428) (width 0.2) (layer "F.Cu") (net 3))
 (segment (start 125.6735 78.4448) (end 122.6183 81.5) (width 0.2) (layer "F.Cu") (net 3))
 (segment (start 166.7098 90.9344) (end 165.977 90.9344) (width 0.2) (layer "F.Cu") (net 3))
 (segment (start 165.977 90.9344) (end 166.7098 90.9344) (width 0.2) (layer "F.Cu") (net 3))
 (segment (start 164.707 69.3145) (end 163.6053 69.3145) (width 0.2) (layer "F.Cu") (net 3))
 (segment (start 122.6183 81.5) (end 105.5 81.5) (width 0.2) (layer "F.Cu") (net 3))
 (via (at 166.7098 90.9344) (size 0.6) (drill 0.3) (layers "F.Cu" "B.Cu") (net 3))
 (via (at 126.3244 70.4277) (size 0.6) (drill 0.3) (layers "F.Cu" "B.Cu") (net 3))
 (via (at 125.6735 78.4448) (size 0.6) (drill 0.3) (layers "F.Cu" "B.Cu") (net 3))
 (segment (start 126.3244 55.7156) (end 126.3244 70.4277) (width 0.2) (layer "B.Cu") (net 3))
 (segment (start 113.12 89.12) (end 113.12 89.0787) (width 0.2) (layer "B.Cu") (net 3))
 (segment (start 113.12 89.0787) (end 113.12 81.5) (width 0.2) (layer "B.Cu") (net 3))
 (segment (start 105.5 81.5) (end 113.12 81.5) (width 0.2) (layer "B.Cu") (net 3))
 (segment (start 113.12 94.2) (end 113.12 89.12) (width 0.2) (layer "B.Cu") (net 3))
 (segment (start 164.707 69.3145) (end 164.707 70.4162) (width 0.2) (layer "B.Cu") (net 3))
 (segment (start 165.8087 71.5179) (end 165.8087 90.0333) (width 0.2) (layer "B.Cu") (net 3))
 (segment (start 128 54.04) (end 126.3244 55.7156) (width 0.2) (layer "B.Cu") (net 3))
 (segment (start 125.6735 71.0786) (end 125.6735 78.4448) (width 0.2) (layer "B.Cu") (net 3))
 (segment (start 164.707 70.4162) (end 165.8087 71.5179) (width 0.2) (layer "B.Cu") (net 3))
 (segment (start 165.977 90.9344) (end 166.7098 90.9344) (width 0.2) (layer "B.Cu") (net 3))
 (segment (start 126.3244 70.4277) (end 125.6735 71.0786) (width 0.2) (layer "B.Cu") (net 3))
 (segment (start 166.7098 90.9344) (end 165.977 90.9344) (width 0.2) (layer "B.Cu") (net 3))
 (segment (start 165.8087 90.0333) (end 166.7098 90.9344) (width 0.2) (layer "B.Cu") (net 3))
 (segment (start 180.8862 63.2176) (end 178.423 60.7544) (width 0.2) (layer "F.Cu") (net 11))
 (segment (start 178.423 60.7544) (end 180.8862 63.2176) (width 0.2) (layer "F.Cu") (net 11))
 (segment (start 180.8862 63.2176) (end 176.7886 59.12) (width 0.2) (layer "F.Cu") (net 11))
 (segment (start 176.7886 59.12) (end 128 59.12) (width 0.2) (layer "F.Cu") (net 11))
 (via (at 180.8862 63.2176) (size 0.6) (drill 0.3) (layers "F.Cu" "B.Cu") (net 11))
 (segment (start 180.8862 63.2176) (end 178.423 60.7544) (width 0.2) (layer "B.Cu") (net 11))
 (segment (start 183.5982 70.7605) (end 183.5982 65.9296) (width 0.2) (layer "B.Cu") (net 11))
 (segment (start 178.423 60.7544) (end 180.8862 63.2176) (width 0.2) (layer "B.Cu") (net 11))
 (segment (start 182.487 84.5545) (end 182.487 71.8717) (width 0.2) (layer "B.Cu") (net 11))
 (segment (start 183.5982 65.9296) (end 180.8862 63.2176) (width 0.2) (layer "B.Cu") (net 11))
 (segment (start 182.487 71.8717) (end 183.5982 70.7605) (width 0.2) (layer "B.Cu") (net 11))
 (segment (start 182.5967 54.4032) (end 182.5967 46.6582) (width 0.2) (layer "B.Cu") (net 32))
 (segment (start 182.6517 54.4582) (end 182.5967 54.4032) (width 0.2) (layer "B.Cu") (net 32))
 (segment (start 186.9 99.835) (end 120.2005 99.835) (width 0.2) (layer "F.Cu") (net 7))
 (segment (start 119.5562 99.1907) (end 120.2005 99.835) (width 0.2) (layer "F.Cu") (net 7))
 (segment (start 120.2005 99.835) (end 119.5562 99.1907) (width 0.2) (layer "F.Cu") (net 7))
 (segment (start 120.2005 99.835) (end 119.5562 99.1907) (width 0.2) (layer "F.Cu") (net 7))
 (via (at 119.5562 99.1907) (size 0.6) (drill 0.3) (layers "F.Cu" "B.Cu") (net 7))
 (segment (start 119.5562 99.1907) (end 120.2005 99.835) (width 0.2) (layer "B.Cu") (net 7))
 (segment (start 119.5562 99.1907) (end 119.5562 79.0642) (width 0.2) (layer "B.Cu") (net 7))
 (segment (start 116.58 76.088) (end 116.58 64.5) (width 0.2) (layer "B.Cu") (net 7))
 (segment (start 120.2005 99.835) (end 119.5562 99.1907) (width 0.2) (layer "B.Cu") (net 7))
 (segment (start 119.5562 79.0642) (end 116.58 76.088) (width 0.2) (layer "B.Cu") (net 7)))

